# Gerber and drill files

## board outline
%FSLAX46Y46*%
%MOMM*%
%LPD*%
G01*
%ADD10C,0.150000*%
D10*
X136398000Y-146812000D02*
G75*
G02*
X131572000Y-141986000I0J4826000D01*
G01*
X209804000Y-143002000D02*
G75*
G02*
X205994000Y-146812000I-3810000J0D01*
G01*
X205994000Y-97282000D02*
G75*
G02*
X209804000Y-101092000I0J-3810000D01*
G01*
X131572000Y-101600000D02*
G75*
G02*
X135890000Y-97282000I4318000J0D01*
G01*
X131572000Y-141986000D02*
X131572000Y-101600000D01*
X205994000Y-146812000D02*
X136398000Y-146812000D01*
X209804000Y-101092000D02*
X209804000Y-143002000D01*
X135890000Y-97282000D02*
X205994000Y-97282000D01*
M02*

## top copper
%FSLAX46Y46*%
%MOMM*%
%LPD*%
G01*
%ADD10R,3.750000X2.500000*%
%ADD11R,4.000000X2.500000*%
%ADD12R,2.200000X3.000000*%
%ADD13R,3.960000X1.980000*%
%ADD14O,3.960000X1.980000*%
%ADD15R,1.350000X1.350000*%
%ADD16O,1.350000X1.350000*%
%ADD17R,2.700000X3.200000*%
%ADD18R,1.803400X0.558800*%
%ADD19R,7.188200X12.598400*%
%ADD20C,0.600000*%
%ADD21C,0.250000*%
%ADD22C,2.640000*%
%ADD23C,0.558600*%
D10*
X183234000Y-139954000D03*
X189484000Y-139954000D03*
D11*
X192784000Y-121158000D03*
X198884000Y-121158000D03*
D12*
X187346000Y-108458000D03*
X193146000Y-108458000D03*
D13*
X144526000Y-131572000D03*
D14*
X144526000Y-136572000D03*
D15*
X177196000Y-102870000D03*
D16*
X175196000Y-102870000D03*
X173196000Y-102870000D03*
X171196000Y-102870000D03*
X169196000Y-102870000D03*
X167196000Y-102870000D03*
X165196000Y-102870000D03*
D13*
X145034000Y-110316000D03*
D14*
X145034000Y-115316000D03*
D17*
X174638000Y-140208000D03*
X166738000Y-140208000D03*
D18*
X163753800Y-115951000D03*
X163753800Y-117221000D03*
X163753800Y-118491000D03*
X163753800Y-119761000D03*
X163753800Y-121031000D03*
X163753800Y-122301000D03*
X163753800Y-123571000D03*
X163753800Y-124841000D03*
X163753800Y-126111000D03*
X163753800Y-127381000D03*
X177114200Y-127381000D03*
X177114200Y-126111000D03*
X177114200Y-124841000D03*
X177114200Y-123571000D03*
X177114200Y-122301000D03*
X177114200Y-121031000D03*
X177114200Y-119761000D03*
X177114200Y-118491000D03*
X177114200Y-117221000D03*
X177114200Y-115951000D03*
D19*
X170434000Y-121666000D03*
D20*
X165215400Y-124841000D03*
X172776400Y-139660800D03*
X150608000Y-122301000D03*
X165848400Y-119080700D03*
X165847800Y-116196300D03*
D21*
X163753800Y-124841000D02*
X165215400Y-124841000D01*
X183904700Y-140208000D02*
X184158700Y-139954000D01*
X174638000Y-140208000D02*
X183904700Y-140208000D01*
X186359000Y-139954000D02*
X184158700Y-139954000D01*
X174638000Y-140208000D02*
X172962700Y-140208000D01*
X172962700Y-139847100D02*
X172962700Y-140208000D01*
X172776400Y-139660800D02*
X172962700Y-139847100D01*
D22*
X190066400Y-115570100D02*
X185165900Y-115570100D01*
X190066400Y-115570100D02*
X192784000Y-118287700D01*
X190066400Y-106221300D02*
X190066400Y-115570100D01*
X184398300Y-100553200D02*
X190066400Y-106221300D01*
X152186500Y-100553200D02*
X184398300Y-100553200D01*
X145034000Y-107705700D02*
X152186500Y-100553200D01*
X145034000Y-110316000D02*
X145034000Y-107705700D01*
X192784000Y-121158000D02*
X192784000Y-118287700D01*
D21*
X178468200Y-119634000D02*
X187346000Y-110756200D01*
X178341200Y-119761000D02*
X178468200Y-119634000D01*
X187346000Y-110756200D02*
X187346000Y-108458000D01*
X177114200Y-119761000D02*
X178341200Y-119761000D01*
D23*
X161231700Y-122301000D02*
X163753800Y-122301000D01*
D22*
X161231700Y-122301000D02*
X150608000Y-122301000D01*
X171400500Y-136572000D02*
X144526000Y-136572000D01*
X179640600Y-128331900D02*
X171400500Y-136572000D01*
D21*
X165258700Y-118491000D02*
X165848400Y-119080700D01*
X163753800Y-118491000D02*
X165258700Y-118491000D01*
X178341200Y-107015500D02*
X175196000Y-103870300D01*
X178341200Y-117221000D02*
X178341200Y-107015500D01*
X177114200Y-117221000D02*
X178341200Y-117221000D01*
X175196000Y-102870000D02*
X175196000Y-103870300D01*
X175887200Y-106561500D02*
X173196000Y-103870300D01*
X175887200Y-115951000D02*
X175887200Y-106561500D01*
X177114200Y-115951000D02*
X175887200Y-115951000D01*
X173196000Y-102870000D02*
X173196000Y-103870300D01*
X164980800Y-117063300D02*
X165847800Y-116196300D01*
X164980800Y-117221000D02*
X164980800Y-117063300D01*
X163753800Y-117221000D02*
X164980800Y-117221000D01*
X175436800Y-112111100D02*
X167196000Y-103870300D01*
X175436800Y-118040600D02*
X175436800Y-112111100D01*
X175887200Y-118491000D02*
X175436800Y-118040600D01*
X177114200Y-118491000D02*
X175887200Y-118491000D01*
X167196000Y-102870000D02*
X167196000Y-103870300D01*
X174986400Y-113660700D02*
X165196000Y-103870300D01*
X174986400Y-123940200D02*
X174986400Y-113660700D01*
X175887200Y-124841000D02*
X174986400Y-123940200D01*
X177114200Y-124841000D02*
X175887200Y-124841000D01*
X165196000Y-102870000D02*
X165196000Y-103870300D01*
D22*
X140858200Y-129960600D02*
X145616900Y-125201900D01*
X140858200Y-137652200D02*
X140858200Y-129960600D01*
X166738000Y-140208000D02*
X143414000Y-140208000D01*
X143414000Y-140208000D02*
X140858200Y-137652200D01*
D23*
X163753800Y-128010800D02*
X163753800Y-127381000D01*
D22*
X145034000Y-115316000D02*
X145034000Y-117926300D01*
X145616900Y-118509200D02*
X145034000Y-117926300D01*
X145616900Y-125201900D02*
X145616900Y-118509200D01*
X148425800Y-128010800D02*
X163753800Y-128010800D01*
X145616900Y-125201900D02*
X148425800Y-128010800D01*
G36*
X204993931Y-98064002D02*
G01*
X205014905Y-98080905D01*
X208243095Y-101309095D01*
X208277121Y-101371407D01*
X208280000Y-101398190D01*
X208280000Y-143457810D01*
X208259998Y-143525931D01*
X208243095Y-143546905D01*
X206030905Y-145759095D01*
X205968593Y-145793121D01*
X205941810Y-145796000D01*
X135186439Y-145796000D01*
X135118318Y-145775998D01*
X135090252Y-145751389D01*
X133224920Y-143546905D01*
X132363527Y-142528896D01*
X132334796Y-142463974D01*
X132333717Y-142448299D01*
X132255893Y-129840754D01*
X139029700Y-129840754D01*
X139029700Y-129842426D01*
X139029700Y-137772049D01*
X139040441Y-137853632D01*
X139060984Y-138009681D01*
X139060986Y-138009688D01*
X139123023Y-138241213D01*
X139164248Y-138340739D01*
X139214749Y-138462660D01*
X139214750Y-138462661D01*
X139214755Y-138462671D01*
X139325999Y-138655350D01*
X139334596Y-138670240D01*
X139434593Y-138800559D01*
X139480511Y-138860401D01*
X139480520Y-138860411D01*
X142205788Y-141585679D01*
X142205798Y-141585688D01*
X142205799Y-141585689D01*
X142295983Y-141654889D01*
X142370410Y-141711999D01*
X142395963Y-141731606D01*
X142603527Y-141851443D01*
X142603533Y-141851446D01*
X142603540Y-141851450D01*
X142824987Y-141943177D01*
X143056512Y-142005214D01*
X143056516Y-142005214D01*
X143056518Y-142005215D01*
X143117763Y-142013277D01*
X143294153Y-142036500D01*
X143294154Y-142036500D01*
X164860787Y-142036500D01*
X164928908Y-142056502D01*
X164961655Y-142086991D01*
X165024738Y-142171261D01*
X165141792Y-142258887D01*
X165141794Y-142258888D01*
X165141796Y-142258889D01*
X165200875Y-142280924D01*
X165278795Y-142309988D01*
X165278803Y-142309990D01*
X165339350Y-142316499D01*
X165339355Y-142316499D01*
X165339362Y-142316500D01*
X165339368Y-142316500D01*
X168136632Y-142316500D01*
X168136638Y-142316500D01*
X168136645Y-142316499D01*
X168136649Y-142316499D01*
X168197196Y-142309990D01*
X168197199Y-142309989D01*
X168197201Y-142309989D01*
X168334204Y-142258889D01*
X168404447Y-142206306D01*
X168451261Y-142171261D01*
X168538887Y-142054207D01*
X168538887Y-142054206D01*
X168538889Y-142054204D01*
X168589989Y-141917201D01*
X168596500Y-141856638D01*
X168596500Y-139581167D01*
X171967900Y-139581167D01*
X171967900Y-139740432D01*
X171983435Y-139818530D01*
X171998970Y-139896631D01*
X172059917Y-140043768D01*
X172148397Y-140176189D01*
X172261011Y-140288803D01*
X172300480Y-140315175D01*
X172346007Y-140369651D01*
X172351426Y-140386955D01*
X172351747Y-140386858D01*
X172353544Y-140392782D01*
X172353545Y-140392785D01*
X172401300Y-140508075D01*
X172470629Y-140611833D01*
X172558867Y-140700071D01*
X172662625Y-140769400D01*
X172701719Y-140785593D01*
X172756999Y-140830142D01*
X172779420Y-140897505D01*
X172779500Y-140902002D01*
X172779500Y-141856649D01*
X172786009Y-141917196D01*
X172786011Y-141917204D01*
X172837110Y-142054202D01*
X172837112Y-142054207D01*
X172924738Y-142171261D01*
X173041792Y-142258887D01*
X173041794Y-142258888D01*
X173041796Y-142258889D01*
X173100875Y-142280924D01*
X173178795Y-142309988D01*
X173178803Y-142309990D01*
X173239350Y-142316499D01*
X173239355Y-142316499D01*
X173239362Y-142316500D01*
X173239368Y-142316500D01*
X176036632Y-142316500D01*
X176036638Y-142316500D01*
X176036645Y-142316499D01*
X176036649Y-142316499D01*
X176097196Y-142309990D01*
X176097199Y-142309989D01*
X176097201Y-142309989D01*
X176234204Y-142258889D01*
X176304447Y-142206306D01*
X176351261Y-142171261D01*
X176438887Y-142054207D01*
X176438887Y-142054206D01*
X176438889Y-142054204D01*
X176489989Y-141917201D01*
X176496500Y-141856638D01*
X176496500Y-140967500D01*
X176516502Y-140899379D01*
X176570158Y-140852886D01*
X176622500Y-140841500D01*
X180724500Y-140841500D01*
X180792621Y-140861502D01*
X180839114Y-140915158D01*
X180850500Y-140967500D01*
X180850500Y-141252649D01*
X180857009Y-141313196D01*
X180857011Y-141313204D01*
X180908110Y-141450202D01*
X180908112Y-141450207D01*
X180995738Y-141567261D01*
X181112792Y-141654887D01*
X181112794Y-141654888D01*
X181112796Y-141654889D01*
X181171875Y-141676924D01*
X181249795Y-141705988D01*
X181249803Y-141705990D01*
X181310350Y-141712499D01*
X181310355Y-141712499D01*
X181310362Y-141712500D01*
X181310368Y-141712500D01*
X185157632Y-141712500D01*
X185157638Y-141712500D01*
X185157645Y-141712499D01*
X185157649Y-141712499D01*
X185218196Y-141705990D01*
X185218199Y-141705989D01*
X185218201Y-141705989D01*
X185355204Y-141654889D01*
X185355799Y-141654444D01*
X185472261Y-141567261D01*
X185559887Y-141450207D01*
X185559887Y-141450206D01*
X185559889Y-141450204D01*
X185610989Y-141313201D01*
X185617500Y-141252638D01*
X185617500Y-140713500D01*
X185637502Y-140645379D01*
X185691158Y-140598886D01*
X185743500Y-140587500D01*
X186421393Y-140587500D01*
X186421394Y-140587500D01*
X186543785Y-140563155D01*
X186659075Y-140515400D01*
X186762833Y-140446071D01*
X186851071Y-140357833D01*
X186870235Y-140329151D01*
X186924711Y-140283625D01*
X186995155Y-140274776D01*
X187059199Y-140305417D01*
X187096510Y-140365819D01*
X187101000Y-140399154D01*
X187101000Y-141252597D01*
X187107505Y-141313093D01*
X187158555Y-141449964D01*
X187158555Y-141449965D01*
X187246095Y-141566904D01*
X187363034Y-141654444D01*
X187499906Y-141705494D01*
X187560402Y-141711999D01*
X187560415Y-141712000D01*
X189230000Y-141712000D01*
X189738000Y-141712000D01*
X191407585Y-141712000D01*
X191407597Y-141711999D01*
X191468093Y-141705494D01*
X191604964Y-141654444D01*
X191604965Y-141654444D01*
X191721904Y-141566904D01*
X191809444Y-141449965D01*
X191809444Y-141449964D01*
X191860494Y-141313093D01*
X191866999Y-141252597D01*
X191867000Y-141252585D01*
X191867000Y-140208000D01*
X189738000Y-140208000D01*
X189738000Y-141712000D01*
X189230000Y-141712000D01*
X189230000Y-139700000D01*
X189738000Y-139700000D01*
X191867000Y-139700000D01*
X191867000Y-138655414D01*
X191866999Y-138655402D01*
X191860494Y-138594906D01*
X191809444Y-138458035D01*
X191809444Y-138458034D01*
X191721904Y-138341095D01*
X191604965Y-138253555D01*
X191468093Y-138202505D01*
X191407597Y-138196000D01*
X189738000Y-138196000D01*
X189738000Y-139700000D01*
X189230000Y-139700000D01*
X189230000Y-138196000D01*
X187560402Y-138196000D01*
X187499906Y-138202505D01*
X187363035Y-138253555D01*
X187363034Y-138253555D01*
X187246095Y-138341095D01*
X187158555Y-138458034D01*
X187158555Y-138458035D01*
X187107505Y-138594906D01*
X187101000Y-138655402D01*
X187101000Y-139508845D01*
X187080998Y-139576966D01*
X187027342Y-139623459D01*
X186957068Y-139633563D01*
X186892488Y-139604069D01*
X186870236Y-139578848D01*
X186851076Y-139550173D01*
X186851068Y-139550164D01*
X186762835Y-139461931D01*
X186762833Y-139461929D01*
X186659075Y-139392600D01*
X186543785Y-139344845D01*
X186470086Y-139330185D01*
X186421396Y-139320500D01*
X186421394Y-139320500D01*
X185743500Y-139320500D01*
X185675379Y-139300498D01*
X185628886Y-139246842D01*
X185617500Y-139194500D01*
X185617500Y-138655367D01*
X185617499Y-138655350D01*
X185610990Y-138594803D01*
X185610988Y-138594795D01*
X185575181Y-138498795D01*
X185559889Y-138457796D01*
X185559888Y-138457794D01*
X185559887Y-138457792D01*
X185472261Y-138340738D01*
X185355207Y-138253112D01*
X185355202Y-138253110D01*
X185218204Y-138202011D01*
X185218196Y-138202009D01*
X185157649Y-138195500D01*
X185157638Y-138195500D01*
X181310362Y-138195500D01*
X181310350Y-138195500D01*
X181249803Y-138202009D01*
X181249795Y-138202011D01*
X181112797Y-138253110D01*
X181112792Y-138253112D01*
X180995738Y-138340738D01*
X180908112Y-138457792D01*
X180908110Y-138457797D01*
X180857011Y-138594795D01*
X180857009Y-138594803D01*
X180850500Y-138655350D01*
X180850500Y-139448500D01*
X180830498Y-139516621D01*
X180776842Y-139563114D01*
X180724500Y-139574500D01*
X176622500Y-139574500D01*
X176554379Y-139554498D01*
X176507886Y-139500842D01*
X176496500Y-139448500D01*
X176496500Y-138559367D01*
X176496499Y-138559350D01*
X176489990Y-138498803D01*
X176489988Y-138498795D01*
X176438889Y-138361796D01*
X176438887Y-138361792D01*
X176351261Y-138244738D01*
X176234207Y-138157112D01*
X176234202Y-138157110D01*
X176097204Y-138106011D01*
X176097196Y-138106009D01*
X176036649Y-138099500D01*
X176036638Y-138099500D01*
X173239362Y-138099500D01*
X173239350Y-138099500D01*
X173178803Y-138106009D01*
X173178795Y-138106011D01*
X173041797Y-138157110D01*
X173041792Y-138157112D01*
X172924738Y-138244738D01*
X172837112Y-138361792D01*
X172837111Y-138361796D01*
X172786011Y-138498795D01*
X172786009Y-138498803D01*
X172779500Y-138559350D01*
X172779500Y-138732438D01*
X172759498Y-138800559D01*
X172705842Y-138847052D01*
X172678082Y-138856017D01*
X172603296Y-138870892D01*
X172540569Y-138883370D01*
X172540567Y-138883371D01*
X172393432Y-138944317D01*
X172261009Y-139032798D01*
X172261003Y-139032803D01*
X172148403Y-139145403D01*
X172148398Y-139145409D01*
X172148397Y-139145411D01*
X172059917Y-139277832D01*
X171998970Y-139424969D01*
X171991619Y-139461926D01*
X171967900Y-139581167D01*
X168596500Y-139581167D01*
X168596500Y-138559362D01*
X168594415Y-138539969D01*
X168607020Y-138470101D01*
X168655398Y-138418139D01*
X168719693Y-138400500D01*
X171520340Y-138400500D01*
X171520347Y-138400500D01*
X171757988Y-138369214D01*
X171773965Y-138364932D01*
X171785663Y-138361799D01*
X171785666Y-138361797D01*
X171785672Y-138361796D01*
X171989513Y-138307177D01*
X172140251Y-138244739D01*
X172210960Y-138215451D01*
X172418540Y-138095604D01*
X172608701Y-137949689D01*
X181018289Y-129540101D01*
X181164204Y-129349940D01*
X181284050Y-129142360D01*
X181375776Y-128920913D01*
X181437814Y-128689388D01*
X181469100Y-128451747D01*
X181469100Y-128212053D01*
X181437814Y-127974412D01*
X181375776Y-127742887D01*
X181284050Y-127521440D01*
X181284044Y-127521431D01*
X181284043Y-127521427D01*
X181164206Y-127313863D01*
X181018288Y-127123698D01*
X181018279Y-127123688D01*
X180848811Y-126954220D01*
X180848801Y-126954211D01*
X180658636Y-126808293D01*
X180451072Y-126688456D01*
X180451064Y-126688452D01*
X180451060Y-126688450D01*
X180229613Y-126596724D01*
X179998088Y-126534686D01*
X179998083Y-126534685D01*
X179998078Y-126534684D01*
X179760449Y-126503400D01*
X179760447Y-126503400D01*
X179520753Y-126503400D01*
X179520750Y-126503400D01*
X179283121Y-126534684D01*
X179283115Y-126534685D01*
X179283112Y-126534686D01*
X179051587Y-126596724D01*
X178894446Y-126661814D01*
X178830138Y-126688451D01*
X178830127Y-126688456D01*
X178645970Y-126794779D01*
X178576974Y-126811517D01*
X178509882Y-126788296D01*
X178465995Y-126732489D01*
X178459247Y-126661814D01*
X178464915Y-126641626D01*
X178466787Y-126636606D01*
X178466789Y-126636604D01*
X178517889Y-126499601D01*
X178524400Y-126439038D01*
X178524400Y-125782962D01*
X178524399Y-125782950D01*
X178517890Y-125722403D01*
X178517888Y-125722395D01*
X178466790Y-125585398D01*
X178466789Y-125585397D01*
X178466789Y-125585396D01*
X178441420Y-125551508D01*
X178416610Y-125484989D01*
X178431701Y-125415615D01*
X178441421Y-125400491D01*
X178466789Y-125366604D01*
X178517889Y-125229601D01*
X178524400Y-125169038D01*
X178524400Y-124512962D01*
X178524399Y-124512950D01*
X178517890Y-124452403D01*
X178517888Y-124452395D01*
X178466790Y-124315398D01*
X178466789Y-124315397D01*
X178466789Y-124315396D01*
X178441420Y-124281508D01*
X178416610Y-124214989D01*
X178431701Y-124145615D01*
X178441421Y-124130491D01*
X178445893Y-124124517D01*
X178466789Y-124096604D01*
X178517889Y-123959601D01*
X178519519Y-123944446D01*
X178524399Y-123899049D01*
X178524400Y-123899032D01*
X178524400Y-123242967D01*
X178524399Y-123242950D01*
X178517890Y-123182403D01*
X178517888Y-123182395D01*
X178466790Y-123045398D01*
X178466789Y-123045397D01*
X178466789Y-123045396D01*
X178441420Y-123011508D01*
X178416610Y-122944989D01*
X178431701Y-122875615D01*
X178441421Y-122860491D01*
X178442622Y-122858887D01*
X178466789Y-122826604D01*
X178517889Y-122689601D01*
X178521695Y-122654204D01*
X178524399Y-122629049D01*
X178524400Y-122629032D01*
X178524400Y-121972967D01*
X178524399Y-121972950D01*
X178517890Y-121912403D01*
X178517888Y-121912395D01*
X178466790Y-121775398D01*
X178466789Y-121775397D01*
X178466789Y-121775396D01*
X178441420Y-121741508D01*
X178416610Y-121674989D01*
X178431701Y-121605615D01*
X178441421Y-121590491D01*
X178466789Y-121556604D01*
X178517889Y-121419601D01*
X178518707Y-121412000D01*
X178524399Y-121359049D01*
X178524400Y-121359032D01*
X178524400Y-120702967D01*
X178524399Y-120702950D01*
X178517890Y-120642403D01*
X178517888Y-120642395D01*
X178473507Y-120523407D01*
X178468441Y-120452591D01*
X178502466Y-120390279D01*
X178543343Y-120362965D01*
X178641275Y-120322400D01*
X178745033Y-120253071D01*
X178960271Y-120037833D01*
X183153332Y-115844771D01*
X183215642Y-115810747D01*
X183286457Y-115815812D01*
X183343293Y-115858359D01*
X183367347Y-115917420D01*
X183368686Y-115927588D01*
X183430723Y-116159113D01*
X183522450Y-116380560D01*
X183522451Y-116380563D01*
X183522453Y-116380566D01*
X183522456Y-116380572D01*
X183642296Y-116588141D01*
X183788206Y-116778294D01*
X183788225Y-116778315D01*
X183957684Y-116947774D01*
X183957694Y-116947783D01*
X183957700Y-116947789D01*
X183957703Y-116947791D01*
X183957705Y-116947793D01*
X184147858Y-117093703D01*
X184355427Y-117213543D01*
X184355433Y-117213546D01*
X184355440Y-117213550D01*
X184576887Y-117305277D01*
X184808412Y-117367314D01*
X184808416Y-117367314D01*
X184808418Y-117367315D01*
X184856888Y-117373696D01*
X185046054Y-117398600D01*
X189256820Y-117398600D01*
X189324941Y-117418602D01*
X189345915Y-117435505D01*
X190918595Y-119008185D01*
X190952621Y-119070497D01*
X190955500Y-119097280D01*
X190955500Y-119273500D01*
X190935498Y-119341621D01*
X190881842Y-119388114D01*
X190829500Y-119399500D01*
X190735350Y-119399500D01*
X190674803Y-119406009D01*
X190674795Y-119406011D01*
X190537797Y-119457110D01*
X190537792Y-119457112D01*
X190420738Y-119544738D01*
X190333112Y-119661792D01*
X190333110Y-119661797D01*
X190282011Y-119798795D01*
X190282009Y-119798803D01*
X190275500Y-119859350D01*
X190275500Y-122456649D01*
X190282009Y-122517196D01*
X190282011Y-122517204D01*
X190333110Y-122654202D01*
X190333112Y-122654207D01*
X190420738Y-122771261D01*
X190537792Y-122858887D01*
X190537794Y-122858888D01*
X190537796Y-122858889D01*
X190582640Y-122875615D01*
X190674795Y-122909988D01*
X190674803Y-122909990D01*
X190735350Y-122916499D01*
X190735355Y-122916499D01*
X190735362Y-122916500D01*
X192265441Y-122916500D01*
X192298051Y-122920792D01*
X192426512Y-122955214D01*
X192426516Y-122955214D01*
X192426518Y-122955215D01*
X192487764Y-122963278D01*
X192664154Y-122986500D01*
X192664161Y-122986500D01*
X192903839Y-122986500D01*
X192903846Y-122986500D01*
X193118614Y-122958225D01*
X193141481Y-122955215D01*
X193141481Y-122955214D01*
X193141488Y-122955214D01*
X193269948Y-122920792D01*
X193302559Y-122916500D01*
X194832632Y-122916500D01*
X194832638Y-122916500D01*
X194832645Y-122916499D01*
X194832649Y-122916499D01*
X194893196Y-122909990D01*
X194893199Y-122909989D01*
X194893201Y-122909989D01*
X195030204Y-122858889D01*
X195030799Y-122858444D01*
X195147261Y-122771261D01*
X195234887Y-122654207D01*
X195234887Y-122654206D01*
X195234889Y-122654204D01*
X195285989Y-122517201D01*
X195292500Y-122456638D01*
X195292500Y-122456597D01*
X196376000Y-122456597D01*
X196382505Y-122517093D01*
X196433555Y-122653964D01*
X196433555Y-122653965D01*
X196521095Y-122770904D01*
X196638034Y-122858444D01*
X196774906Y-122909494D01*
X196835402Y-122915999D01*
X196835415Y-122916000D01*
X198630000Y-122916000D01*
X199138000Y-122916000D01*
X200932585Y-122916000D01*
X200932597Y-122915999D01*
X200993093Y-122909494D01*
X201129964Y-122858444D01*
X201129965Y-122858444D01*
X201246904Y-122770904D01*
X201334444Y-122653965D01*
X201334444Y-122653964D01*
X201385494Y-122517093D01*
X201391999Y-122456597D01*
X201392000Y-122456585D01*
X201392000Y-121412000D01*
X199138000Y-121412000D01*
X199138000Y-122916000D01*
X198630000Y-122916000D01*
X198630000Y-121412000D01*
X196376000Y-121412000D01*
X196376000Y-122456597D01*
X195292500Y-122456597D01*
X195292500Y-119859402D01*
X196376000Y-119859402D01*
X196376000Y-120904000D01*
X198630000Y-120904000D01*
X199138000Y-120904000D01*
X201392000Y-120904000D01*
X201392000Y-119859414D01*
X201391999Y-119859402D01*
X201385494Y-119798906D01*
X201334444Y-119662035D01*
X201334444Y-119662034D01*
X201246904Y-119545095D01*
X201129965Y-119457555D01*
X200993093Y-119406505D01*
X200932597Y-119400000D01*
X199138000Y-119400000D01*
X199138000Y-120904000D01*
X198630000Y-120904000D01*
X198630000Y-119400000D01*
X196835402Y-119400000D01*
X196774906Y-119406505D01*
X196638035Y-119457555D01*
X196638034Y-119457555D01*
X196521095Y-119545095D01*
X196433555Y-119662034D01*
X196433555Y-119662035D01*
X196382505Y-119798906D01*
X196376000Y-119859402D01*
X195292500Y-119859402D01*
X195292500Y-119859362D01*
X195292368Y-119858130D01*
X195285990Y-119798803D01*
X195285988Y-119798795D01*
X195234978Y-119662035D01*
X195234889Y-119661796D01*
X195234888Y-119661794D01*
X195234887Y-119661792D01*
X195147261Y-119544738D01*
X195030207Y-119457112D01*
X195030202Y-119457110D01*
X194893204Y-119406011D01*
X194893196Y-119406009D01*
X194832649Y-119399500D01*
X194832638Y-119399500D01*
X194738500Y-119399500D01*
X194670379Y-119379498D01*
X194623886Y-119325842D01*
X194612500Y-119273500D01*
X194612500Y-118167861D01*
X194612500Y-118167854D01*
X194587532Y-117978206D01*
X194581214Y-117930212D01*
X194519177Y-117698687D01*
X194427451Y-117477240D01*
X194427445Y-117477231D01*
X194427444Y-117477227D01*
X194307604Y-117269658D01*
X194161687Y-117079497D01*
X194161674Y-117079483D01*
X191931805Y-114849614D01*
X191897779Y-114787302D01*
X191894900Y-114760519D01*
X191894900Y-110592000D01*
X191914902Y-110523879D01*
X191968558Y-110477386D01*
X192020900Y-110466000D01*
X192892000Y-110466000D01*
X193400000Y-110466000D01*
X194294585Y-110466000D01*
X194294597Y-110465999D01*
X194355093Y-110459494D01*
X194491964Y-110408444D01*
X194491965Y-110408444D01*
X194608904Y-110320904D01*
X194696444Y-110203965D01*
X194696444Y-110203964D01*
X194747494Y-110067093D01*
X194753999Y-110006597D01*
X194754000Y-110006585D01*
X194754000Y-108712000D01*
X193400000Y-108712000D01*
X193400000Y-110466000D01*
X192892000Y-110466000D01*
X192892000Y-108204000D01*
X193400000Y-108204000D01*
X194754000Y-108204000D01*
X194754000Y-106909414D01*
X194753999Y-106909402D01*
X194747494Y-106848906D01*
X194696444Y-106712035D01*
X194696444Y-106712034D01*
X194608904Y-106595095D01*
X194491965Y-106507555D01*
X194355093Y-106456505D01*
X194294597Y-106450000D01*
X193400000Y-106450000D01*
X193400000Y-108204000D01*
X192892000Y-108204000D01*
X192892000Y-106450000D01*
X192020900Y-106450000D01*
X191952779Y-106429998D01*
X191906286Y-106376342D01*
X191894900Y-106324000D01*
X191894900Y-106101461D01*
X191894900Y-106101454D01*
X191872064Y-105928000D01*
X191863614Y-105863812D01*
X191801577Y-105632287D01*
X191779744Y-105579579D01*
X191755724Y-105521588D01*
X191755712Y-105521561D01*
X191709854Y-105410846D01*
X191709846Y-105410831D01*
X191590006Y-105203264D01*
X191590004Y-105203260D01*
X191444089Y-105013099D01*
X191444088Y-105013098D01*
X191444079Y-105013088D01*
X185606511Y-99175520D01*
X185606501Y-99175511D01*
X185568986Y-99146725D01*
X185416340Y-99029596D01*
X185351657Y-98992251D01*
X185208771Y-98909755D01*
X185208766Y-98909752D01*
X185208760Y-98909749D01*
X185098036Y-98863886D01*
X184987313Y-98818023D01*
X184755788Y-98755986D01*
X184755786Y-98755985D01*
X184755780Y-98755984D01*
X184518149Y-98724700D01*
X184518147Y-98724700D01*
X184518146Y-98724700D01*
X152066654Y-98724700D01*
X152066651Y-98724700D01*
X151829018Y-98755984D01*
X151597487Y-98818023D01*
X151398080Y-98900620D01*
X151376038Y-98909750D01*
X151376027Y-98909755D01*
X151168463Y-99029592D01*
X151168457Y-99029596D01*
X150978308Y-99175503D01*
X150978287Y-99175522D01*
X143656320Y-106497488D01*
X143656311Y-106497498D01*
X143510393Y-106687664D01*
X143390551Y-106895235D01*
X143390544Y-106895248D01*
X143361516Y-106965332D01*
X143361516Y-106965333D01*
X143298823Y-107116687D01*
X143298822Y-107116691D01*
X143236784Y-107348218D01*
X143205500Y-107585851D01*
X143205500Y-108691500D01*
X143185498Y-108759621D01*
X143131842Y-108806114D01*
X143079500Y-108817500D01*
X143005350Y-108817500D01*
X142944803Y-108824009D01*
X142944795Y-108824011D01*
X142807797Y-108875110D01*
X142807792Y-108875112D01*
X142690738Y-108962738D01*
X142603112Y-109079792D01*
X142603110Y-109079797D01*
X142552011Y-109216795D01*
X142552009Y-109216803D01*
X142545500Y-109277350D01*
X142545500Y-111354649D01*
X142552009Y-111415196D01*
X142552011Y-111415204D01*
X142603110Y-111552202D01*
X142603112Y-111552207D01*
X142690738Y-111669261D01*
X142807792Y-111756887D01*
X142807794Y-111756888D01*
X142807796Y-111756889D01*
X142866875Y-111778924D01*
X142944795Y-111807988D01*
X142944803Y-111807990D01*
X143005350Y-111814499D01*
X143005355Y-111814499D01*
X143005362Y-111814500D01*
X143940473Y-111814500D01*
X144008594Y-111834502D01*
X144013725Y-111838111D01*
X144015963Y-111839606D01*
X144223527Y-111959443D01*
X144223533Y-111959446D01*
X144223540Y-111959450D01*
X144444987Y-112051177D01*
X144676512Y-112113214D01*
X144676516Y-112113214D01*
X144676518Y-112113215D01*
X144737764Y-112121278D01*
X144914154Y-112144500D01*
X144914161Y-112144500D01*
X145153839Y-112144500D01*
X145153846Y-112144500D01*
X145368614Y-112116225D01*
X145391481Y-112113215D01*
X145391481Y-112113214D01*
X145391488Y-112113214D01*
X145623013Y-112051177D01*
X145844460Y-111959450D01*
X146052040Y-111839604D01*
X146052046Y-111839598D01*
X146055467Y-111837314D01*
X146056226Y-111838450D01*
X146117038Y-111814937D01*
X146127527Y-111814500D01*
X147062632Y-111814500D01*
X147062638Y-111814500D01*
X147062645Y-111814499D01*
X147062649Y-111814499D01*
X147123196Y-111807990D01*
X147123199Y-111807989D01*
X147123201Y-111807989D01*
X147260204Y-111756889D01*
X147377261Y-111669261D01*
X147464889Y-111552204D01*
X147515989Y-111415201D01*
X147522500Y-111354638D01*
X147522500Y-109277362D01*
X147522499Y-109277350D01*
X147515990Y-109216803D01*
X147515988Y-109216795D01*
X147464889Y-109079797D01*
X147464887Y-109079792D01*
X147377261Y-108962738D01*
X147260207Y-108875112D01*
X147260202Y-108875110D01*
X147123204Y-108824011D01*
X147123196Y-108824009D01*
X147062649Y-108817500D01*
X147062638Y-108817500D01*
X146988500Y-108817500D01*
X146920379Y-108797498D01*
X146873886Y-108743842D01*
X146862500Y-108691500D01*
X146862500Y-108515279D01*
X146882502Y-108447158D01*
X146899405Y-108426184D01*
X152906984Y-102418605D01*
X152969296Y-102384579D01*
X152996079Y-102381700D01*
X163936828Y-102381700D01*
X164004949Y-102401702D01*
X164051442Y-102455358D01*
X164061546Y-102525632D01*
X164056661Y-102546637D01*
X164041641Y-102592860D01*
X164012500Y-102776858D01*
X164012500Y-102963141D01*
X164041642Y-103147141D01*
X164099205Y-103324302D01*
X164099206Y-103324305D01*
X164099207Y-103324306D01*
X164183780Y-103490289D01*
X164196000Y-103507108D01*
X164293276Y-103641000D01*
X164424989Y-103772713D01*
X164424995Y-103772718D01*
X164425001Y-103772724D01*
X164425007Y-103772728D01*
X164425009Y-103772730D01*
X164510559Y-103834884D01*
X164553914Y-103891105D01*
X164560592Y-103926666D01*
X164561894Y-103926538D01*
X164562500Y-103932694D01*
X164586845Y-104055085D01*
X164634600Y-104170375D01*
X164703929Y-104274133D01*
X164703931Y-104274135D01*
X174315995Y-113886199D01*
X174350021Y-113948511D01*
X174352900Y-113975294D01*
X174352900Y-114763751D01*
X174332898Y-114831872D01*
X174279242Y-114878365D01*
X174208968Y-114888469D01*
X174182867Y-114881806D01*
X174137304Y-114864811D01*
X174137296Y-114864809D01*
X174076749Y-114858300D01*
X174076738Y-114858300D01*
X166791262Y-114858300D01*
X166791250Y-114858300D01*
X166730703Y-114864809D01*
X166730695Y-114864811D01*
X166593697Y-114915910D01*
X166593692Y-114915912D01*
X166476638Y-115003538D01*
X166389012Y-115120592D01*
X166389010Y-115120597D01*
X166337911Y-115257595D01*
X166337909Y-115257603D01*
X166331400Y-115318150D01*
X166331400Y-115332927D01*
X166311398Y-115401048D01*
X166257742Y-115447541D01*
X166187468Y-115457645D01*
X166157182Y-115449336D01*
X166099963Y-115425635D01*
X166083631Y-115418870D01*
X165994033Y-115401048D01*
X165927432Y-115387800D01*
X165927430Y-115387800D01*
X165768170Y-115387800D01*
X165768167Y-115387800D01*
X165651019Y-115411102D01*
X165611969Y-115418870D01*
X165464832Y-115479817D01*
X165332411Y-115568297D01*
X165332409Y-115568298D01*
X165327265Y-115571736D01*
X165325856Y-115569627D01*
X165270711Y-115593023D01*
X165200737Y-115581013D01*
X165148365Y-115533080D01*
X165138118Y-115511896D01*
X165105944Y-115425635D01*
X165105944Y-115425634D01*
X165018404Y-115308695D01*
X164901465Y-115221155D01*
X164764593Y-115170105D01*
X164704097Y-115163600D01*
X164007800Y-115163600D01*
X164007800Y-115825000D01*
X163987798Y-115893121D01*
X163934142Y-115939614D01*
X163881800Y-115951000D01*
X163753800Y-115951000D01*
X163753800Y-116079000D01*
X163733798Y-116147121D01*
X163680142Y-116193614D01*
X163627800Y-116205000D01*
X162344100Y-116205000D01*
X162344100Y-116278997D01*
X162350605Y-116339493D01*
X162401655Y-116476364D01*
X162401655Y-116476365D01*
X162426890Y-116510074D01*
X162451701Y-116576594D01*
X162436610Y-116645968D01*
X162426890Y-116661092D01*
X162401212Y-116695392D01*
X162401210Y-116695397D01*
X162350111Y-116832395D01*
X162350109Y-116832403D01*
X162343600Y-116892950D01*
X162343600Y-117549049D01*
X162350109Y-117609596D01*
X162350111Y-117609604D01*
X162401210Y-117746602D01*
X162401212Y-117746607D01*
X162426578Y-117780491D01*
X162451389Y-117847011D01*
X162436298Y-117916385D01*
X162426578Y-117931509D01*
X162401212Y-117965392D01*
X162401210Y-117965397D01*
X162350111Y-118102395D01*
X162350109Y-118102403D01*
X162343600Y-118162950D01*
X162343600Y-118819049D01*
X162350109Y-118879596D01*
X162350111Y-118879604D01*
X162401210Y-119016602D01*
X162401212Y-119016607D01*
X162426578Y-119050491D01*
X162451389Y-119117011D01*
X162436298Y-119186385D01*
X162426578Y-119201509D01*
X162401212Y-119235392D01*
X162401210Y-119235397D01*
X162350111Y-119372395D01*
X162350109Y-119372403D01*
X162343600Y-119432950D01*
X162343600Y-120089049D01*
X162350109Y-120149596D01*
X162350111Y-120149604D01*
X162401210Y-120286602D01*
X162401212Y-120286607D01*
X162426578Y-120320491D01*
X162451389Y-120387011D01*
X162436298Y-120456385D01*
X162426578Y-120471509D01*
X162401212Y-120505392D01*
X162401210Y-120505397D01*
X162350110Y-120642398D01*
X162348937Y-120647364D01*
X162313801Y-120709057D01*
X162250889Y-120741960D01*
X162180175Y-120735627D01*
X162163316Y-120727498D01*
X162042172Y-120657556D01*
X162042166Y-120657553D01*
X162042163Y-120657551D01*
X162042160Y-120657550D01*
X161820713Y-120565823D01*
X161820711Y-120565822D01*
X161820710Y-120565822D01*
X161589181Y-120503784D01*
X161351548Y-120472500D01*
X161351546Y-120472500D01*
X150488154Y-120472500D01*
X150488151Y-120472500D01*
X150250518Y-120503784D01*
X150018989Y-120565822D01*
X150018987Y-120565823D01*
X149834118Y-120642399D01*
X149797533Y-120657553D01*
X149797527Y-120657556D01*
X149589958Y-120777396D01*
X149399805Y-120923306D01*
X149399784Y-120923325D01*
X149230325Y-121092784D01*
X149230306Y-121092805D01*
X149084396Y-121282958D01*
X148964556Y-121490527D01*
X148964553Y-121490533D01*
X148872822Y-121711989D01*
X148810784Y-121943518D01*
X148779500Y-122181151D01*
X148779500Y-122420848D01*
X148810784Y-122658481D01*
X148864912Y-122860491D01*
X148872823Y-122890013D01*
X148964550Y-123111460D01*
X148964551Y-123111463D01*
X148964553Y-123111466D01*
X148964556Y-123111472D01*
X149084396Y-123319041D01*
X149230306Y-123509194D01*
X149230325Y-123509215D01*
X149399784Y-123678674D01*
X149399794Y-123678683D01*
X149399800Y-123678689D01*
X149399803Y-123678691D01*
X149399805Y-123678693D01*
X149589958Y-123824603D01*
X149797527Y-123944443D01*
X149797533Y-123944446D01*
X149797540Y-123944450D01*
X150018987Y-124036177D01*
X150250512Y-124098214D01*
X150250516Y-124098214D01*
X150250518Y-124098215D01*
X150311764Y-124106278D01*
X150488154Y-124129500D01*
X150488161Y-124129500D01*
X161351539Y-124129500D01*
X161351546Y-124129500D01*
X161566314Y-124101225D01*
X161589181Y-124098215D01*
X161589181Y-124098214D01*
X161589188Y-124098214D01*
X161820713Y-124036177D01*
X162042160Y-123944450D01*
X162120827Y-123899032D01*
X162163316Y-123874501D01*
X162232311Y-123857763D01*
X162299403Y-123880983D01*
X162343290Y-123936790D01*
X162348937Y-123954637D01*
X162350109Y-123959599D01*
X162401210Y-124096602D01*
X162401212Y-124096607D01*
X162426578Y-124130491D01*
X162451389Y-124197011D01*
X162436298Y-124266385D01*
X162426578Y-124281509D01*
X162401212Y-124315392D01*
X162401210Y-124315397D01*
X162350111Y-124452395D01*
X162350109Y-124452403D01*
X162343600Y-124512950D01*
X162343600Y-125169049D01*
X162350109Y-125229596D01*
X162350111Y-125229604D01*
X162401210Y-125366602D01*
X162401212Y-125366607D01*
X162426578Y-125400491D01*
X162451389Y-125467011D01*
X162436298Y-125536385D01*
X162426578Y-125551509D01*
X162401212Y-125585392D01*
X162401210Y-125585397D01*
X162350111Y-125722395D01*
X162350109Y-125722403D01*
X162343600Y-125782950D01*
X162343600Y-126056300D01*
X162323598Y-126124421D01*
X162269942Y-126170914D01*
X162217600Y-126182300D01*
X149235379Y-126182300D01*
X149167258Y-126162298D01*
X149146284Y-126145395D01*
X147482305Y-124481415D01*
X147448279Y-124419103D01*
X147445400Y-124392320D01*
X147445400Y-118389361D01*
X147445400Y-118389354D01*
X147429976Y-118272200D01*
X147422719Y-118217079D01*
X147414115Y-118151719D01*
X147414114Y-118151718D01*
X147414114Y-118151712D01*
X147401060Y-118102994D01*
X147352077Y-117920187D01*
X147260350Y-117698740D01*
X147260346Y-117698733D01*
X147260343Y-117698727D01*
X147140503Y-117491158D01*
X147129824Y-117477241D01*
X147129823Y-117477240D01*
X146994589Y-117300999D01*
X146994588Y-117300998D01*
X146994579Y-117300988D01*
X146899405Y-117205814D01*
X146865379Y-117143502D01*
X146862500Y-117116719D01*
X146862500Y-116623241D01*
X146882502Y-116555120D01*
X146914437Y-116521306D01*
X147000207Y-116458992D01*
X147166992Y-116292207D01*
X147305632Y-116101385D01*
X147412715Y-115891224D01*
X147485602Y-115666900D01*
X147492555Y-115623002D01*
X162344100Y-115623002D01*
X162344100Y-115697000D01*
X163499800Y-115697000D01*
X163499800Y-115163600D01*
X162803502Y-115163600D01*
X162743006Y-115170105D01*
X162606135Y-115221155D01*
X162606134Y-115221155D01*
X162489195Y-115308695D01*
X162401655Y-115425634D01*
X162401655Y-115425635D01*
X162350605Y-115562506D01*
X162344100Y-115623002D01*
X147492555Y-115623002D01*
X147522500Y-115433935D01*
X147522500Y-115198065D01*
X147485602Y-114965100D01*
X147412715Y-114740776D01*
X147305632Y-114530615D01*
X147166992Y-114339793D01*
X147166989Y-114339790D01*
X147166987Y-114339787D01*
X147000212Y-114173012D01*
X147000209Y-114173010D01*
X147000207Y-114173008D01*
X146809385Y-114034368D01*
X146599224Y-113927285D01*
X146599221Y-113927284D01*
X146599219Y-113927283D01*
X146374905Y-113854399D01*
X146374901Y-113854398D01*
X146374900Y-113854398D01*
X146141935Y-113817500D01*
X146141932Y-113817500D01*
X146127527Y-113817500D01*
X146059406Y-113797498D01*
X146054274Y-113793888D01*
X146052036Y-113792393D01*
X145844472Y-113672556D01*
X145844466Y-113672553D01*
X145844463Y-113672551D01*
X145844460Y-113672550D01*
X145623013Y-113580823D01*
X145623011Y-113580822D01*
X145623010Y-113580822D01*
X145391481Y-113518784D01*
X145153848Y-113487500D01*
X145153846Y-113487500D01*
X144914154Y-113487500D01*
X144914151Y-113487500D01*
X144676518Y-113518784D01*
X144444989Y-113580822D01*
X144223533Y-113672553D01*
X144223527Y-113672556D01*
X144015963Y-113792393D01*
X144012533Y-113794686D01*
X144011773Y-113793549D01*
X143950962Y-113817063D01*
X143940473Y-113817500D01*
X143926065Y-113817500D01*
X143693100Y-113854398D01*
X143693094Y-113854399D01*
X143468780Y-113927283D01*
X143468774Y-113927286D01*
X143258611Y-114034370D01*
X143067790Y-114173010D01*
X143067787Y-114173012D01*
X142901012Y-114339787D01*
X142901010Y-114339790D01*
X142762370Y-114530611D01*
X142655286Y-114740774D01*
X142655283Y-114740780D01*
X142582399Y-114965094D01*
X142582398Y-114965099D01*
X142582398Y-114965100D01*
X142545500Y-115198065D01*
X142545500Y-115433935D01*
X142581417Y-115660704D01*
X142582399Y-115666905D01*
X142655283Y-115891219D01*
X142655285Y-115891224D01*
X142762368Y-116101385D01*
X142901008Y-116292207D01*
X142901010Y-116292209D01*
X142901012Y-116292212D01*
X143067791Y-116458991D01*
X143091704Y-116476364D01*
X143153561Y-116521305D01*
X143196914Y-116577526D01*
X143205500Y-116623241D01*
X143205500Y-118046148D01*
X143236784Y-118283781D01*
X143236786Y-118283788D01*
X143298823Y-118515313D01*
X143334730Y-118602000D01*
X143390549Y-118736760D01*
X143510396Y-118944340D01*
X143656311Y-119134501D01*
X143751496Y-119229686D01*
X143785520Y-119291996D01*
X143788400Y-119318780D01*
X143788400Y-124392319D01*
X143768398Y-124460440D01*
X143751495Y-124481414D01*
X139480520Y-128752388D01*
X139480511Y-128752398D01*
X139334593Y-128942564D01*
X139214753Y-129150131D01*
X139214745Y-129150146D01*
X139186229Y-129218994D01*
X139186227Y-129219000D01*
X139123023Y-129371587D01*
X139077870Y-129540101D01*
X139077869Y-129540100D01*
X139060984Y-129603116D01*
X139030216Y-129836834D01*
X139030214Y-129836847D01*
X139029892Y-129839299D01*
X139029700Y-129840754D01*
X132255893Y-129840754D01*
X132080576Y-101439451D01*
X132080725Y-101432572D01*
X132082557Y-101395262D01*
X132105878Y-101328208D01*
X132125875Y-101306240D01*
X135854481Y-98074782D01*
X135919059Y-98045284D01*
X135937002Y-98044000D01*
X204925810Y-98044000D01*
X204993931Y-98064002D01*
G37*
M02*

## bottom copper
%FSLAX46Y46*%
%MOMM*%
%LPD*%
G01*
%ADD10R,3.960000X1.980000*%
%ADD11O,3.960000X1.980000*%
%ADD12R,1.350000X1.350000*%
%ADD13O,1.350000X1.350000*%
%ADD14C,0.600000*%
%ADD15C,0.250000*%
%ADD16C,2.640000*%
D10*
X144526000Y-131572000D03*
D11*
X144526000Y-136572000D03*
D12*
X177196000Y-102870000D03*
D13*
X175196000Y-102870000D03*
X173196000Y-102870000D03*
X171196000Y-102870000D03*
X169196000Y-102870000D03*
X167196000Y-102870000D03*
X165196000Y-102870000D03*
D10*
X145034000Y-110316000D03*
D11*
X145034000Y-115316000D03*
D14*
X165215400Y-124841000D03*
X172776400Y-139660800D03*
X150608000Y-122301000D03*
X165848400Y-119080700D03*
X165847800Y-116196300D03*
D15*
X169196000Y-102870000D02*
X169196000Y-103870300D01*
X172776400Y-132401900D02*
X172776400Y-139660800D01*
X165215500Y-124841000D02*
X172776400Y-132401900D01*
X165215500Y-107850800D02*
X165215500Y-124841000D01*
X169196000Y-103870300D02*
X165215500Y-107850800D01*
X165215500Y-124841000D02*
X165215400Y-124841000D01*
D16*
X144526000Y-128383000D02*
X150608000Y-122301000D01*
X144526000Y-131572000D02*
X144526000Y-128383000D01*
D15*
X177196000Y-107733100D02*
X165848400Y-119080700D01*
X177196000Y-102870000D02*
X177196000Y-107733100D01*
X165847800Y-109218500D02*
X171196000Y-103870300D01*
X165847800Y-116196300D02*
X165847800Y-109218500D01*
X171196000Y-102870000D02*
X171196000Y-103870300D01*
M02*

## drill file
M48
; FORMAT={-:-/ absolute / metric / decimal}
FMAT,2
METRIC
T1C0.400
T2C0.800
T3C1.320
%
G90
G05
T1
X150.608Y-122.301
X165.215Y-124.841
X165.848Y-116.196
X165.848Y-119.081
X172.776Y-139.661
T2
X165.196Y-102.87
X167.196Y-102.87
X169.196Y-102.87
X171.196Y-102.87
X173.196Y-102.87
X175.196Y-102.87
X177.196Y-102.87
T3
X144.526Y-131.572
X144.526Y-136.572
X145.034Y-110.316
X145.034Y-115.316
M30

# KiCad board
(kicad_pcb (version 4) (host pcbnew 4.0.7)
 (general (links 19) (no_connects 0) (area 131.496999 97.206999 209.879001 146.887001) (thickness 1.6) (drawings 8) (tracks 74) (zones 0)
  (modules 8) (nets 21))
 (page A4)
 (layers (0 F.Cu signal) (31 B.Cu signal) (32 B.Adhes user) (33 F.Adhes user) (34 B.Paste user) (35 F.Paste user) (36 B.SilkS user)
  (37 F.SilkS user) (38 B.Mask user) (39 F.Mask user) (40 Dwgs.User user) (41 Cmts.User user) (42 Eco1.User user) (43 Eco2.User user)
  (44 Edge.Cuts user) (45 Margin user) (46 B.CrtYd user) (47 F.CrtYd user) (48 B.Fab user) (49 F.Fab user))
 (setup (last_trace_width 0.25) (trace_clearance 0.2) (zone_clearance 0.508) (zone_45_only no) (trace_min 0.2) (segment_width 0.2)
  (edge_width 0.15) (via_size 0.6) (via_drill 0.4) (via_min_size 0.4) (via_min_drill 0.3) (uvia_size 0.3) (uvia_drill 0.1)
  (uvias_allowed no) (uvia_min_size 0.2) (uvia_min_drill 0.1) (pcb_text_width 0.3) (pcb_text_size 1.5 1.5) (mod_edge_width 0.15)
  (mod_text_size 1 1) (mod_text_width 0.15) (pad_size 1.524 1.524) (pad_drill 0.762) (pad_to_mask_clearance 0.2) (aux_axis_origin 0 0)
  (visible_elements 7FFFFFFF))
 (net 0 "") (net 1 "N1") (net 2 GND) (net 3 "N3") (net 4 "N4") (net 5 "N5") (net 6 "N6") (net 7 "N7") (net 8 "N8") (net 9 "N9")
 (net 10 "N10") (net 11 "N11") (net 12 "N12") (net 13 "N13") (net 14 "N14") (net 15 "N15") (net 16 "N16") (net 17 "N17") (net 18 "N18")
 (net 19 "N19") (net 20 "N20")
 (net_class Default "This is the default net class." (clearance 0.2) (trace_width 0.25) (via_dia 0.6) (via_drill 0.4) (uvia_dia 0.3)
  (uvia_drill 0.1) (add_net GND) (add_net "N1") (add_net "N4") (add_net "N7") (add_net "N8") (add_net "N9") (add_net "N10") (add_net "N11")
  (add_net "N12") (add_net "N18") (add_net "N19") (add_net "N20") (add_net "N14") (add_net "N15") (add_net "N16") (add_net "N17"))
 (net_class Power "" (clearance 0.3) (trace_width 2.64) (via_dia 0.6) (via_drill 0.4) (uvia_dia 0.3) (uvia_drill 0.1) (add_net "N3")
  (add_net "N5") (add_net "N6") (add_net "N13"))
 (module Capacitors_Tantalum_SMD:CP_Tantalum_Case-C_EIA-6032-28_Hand (layer F.Cu) (at 186.359 139.954)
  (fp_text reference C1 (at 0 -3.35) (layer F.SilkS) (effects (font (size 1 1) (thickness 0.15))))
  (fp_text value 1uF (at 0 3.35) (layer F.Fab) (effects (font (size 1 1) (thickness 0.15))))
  (pad 1 smd rect (at -3.125 0) (size 3.75 2.5) (layers F.Cu F.Paste F.Mask) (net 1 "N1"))
  (pad 2 smd rect (at 3.125 0) (size 3.75 2.5) (layers F.Cu F.Paste F.Mask) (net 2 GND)))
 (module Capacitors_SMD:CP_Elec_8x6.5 (layer F.Cu) (at 195.834 121.158)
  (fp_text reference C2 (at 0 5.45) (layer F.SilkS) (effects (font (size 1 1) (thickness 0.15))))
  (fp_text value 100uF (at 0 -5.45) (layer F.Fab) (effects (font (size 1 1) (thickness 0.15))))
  (pad 1 smd rect (at -3.05 0 180) (size 4 2.5) (layers F.Cu F.Paste F.Mask) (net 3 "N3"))
  (pad 2 smd rect (at 3.05 0 180) (size 4 2.5) (layers F.Cu F.Paste F.Mask) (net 2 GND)))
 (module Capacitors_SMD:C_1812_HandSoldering (layer F.Cu) (at 190.246 108.458)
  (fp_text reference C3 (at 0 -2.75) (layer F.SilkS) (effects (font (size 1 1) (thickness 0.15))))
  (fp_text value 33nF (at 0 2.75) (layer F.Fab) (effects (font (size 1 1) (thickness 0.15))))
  (pad 1 smd rect (at -2.9 0) (size 2.2 3) (layers F.Cu F.Paste F.Mask) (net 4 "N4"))
  (pad 2 smd rect (at 2.9 0) (size 2.2 3) (layers F.Cu F.Paste F.Mask) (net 2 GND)))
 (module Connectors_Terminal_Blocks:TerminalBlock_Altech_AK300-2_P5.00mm (layer F.Cu) (at 144.526 131.572 270)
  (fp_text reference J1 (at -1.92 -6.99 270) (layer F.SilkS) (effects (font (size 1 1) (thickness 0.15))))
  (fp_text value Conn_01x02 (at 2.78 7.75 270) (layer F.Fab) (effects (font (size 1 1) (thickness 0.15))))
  (pad 1 thru_hole rect (at 0 0 270) (size 1.98 3.96) (drill 1.32) (layers *.Cu *.Mask) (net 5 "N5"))
  (pad 2 thru_hole oval (at 5 0 270) (size 1.98 3.96) (drill 1.32) (layers *.Cu *.Mask) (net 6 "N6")))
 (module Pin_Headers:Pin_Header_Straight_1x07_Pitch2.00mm (layer F.Cu) (at 177.196 102.87 270)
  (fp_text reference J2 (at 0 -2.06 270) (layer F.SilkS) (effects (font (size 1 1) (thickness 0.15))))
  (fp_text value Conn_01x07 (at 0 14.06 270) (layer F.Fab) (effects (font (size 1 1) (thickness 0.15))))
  (pad 1 thru_hole rect (at 0 0 270) (size 1.35 1.35) (drill 0.8) (layers *.Cu *.Mask) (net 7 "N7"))
  (pad 2 thru_hole oval (at 0 2 270) (size 1.35 1.35) (drill 0.8) (layers *.Cu *.Mask) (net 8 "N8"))
  (pad 3 thru_hole oval (at 0 4 270) (size 1.35 1.35) (drill 0.8) (layers *.Cu *.Mask) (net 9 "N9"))
  (pad 4 thru_hole oval (at 0 6 270) (size 1.35 1.35) (drill 0.8) (layers *.Cu *.Mask) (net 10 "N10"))
  (pad 5 thru_hole oval (at 0 8 270) (size 1.35 1.35) (drill 0.8) (layers *.Cu *.Mask) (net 1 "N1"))
  (pad 6 thru_hole oval (at 0 10 270) (size 1.35 1.35) (drill 0.8) (layers *.Cu *.Mask) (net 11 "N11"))
  (pad 7 thru_hole oval (at 0 12 270) (size 1.35 1.35) (drill 0.8) (layers *.Cu *.Mask) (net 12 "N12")))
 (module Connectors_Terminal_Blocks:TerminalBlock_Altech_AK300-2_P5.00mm (layer F.Cu) (at 145.034 110.316 270)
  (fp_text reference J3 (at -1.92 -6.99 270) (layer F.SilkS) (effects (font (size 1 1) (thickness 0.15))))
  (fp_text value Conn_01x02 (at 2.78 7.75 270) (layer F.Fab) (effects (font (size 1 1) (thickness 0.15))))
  (pad 1 thru_hole rect (at 0 0 270) (size 1.98 3.96) (drill 1.32) (layers *.Cu *.Mask) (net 3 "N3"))
  (pad 2 thru_hole oval (at 5 0 270) (size 1.98 3.96) (drill 1.32) (layers *.Cu *.Mask) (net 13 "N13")))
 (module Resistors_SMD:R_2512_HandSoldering (layer F.Cu) (at 170.688 140.208 180)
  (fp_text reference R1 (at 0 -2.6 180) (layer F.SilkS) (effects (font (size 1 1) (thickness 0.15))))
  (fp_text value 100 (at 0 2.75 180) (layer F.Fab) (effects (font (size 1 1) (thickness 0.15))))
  (pad 1 smd rect (at -3.95 0 180) (size 2.7 3.2) (layers F.Cu F.Paste F.Mask) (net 1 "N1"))
  (pad 2 smd rect (at 3.95 0 180) (size 2.7 3.2) (layers F.Cu F.Paste F.Mask) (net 13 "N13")))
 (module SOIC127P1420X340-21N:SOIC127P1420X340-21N (layer F.Cu) (at 170.434 121.666)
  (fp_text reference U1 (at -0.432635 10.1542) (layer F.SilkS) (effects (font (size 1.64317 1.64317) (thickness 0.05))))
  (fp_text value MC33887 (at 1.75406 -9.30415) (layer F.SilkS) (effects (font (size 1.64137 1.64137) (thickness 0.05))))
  (pad 1 smd rect (at -6.6802 -5.715) (size 1.8034 0.5588) (layers F.Cu F.Paste F.Mask) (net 2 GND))
  (pad 2 smd rect (at -6.6802 -4.445) (size 1.8034 0.5588) (layers F.Cu F.Paste F.Mask) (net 10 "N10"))
  (pad 3 smd rect (at -6.6802 -3.175) (size 1.8034 0.5588) (layers F.Cu F.Paste F.Mask) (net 7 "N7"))
  (pad 4 smd rect (at -6.6802 -1.905) (size 1.8034 0.5588) (layers F.Cu F.Paste F.Mask) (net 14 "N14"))
  (pad 5 smd rect (at -6.6802 -0.635) (size 1.8034 0.5588) (layers F.Cu F.Paste F.Mask) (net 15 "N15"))
  (pad 6 smd rect (at -6.6802 0.635) (size 1.8034 0.5588) (layers F.Cu F.Paste F.Mask) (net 5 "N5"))
  (pad 7 smd rect (at -6.6802 1.905) (size 1.8034 0.5588) (layers F.Cu F.Paste F.Mask) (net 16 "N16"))
  (pad 8 smd rect (at -6.6802 3.175) (size 1.8034 0.5588) (layers F.Cu F.Paste F.Mask) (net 1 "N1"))
  (pad 9 smd rect (at -6.6802 4.445) (size 1.8034 0.5588) (layers F.Cu F.Paste F.Mask) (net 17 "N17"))
  (pad 10 smd rect (at -6.6802 5.715) (size 1.8034 0.5588) (layers F.Cu F.Paste F.Mask) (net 13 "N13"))
  (pad 11 smd rect (at 6.6802 5.715) (size 1.8034 0.5588) (layers F.Cu F.Paste F.Mask) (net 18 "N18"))
  (pad 12 smd rect (at 6.6802 4.445) (size 1.8034 0.5588) (layers F.Cu F.Paste F.Mask) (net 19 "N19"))
  (pad 13 smd rect (at 6.6802 3.175) (size 1.8034 0.5588) (layers F.Cu F.Paste F.Mask) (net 12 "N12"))
  (pad 14 smd rect (at 6.6802 1.905) (size 1.8034 0.5588) (layers F.Cu F.Paste F.Mask) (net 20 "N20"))
  (pad 15 smd rect (at 6.6802 0.635) (size 1.8034 0.5588) (layers F.Cu F.Paste F.Mask) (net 6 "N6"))
  (pad 16 smd rect (at 6.6802 -0.635) (size 1.8034 0.5588) (layers F.Cu F.Paste F.Mask) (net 3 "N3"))
  (pad 17 smd rect (at 6.6802 -1.905) (size 1.8034 0.5588) (layers F.Cu F.Paste F.Mask) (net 4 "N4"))
  (pad 18 smd rect (at 6.6802 -3.175) (size 1.8034 0.5588) (layers F.Cu F.Paste F.Mask) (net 11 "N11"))
  (pad 19 smd rect (at 6.6802 -4.445) (size 1.8034 0.5588) (layers F.Cu F.Paste F.Mask) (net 8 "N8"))
  (pad 20 smd rect (at 6.6802 -5.715) (size 1.8034 0.5588) (layers F.Cu F.Paste F.Mask) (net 9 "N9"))
  (pad 21 smd rect (at 0 0) (size 7.1882 12.5984) (layers F.Cu F.Paste F.Mask)))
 (gr_arc (start 136.398 141.986) (end 136.398 146.812) (angle 90) (layer Edge.Cuts) (width 0.15))
 (gr_arc (start 205.994 143.002) (end 209.804 143.002) (angle 90) (layer Edge.Cuts) (width 0.15))
 (gr_arc (start 205.994 101.092) (end 205.994 97.282) (angle 90) (layer Edge.Cuts) (width 0.15))
 (gr_arc (start 135.89 101.6) (end 131.572 101.6) (angle 90) (layer Edge.Cuts) (width 0.15))
 (gr_line (start 131.572 141.986) (end 131.572 101.6) (layer Edge.Cuts) (width 0.15))
 (gr_line (start 205.994 146.812) (end 136.398 146.812) (layer Edge.Cuts) (width 0.15))
 (gr_line (start 209.804 101.092) (end 209.804 143.002) (layer Edge.Cuts) (width 0.15))
 (gr_line (start 135.89 97.282) (end 205.994 97.282) (layer Edge.Cuts) (width 0.15))
 (via (at 165.2154 124.841) (size 0.6) (layers F.Cu B.Cu) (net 1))
 (via (at 172.7764 139.6608) (size 0.6) (layers F.Cu B.Cu) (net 1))
 (segment (start 169.196 102.87) (end 169.196 103.8703) (width 0.25) (layer B.Cu) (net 1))
 (segment (start 163.7538 124.841) (end 165.2154 124.841) (width 0.25) (layer F.Cu) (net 1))
 (segment (start 183.9047 140.208) (end 184.1587 139.954) (width 0.25) (layer F.Cu) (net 1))
 (segment (start 174.638 140.208) (end 183.9047 140.208) (width 0.25) (layer F.Cu) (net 1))
 (segment (start 186.359 139.954) (end 184.1587 139.954) (width 0.25) (layer F.Cu) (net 1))
 (segment (start 174.638 140.208) (end 172.9627 140.208) (width 0.25) (layer F.Cu) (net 1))
 (segment (start 172.9627 139.8471) (end 172.9627 140.208) (width 0.25) (layer F.Cu) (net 1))
 (segment (start 172.7764 139.6608) (end 172.9627 139.8471) (width 0.25) (layer F.Cu) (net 1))
 (segment (start 172.7764 132.4019) (end 172.7764 139.6608) (width 0.25) (layer B.Cu) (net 1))
 (segment (start 165.2155 124.841) (end 172.7764 132.4019) (width 0.25) (layer B.Cu) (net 1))
 (segment (start 165.2155 107.8508) (end 165.2155 124.841) (width 0.25) (layer B.Cu) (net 1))
 (segment (start 169.196 103.8703) (end 165.2155 107.8508) (width 0.25) (layer B.Cu) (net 1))
 (segment (start 165.2155 124.841) (end 165.2154 124.841) (width 0.25) (layer B.Cu) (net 1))
 (segment (start 190.0664 115.5701) (end 185.1659 115.5701) (width 2.64) (layer F.Cu) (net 3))
 (segment (start 190.0664 115.5701) (end 192.784 118.2877) (width 2.64) (layer F.Cu) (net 3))
 (segment (start 190.0664 106.2213) (end 190.0664 115.5701) (width 2.64) (layer F.Cu) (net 3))
 (segment (start 184.3983 100.5532) (end 190.0664 106.2213) (width 2.64) (layer F.Cu) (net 3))
 (segment (start 152.1865 100.5532) (end 184.3983 100.5532) (width 2.64) (layer F.Cu) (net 3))
 (segment (start 145.034 107.7057) (end 152.1865 100.5532) (width 2.64) (layer F.Cu) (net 3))
 (segment (start 145.034 110.316) (end 145.034 107.7057) (width 2.64) (layer F.Cu) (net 3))
 (segment (start 192.784 121.158) (end 192.784 118.2877) (width 2.64) (layer F.Cu) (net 3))
 (segment (start 178.4682 119.634) (end 187.346 110.7562) (width 0.25) (layer F.Cu) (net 4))
 (segment (start 178.3412 119.761) (end 178.4682 119.634) (width 0.25) (layer F.Cu) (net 4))
 (segment (start 187.346 110.7562) (end 187.346 108.458) (width 0.25) (layer F.Cu) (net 4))
 (segment (start 177.1142 119.761) (end 178.3412 119.761) (width 0.25) (layer F.Cu) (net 4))
 (via (at 150.608 122.301) (size 0.6) (layers F.Cu B.Cu) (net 5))
 (segment (start 161.2317 122.301) (end 163.7538 122.301) (width 0.5586) (layer F.Cu) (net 5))
 (segment (start 144.526 128.383) (end 150.608 122.301) (width 2.64) (layer B.Cu) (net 5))
 (segment (start 144.526 131.572) (end 144.526 128.383) (width 2.64) (layer B.Cu) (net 5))
 (segment (start 161.2317 122.301) (end 150.608 122.301) (width 2.64) (layer F.Cu) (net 5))
 (segment (start 171.4005 136.572) (end 144.526 136.572) (width 2.64) (layer F.Cu) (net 6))
 (segment (start 179.6406 128.3319) (end 171.4005 136.572) (width 2.64) (layer F.Cu) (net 6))
 (via (at 165.8484 119.0807) (size 0.6) (layers F.Cu B.Cu) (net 7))
 (segment (start 177.196 107.7331) (end 165.8484 119.0807) (width 0.25) (layer B.Cu) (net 7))
 (segment (start 177.196 102.87) (end 177.196 107.7331) (width 0.25) (layer B.Cu) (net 7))
 (segment (start 165.2587 118.491) (end 165.8484 119.0807) (width 0.25) (layer F.Cu) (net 7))
 (segment (start 163.7538 118.491) (end 165.2587 118.491) (width 0.25) (layer F.Cu) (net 7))
 (segment (start 178.3412 107.0155) (end 175.196 103.8703) (width 0.25) (layer F.Cu) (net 8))
 (segment (start 178.3412 117.221) (end 178.3412 107.0155) (width 0.25) (layer F.Cu) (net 8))
 (segment (start 177.1142 117.221) (end 178.3412 117.221) (width 0.25) (layer F.Cu) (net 8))
 (segment (start 175.196 102.87) (end 175.196 103.8703) (width 0.25) (layer F.Cu) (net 8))
 (segment (start 175.8872 106.5615) (end 173.196 103.8703) (width 0.25) (layer F.Cu) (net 9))
 (segment (start 175.8872 115.951) (end 175.8872 106.5615) (width 0.25) (layer F.Cu) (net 9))
 (segment (start 177.1142 115.951) (end 175.8872 115.951) (width 0.25) (layer F.Cu) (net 9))
 (segment (start 173.196 102.87) (end 173.196 103.8703) (width 0.25) (layer F.Cu) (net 9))
 (via (at 165.8478 116.1963) (size 0.6) (layers F.Cu B.Cu) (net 10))
 (segment (start 164.9808 117.0633) (end 165.8478 116.1963) (width 0.25) (layer F.Cu) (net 10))
 (segment (start 164.9808 117.221) (end 164.9808 117.0633) (width 0.25) (layer F.Cu) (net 10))
 (segment (start 165.8478 109.2185) (end 171.196 103.8703) (width 0.25) (layer B.Cu) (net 10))
 (segment (start 165.8478 116.1963) (end 165.8478 109.2185) (width 0.25) (layer B.Cu) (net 10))
 (segment (start 163.7538 117.221) (end 164.9808 117.221) (width 0.25) (layer F.Cu) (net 10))
 (segment (start 171.196 102.87) (end 171.196 103.8703) (width 0.25) (layer B.Cu) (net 10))
 (segment (start 175.4368 112.1111) (end 167.196 103.8703) (width 0.25) (layer F.Cu) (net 11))
 (segment (start 175.4368 118.0406) (end 175.4368 112.1111) (width 0.25) (layer F.Cu) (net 11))
 (segment (start 175.8872 118.491) (end 175.4368 118.0406) (width 0.25) (layer F.Cu) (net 11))
 (segment (start 177.1142 118.491) (end 175.8872 118.491) (width 0.25) (layer F.Cu) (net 11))
 (segment (start 167.196 102.87) (end 167.196 103.8703) (width 0.25) (layer F.Cu) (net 11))
 (segment (start 174.9864 113.6607) (end 165.196 103.8703) (width 0.25) (layer F.Cu) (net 12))
 (segment (start 174.9864 123.9402) (end 174.9864 113.6607) (width 0.25) (layer F.Cu) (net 12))
 (segment (start 175.8872 124.841) (end 174.9864 123.9402) (width 0.25) (layer F.Cu) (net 12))
 (segment (start 177.1142 124.841) (end 175.8872 124.841) (width 0.25) (layer F.Cu) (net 12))
 (segment (start 165.196 102.87) (end 165.196 103.8703) (width 0.25) (layer F.Cu) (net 12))
 (segment (start 140.8582 129.9606) (end 145.6169 125.2019) (width 2.64) (layer F.Cu) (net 13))
 (segment (start 140.8582 137.6522) (end 140.8582 129.9606) (width 2.64) (layer F.Cu) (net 13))
 (segment (start 166.738 140.208) (end 143.414 140.208) (width 2.64) (layer F.Cu) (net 13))
 (segment (start 143.414 140.208) (end 140.8582 137.6522) (width 2.64) (layer F.Cu) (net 13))
 (segment (start 163.7538 128.0108) (end 163.7538 127.381) (width 0.5586) (layer F.Cu) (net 13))
 (segment (start 145.034 115.316) (end 145.034 117.9263) (width 2.64) (layer F.Cu) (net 13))
 (segment (start 145.6169 118.5092) (end 145.034 117.9263) (width 2.64) (layer F.Cu) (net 13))
 (segment (start 145.6169 125.2019) (end 145.6169 118.5092) (width 2.64) (layer F.Cu) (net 13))
 (segment (start 148.4258 128.0108) (end 163.7538 128.0108) (width 2.64) (layer F.Cu) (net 13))
 (segment (start 145.6169 125.2019) (end 148.4258 128.0108) (width 2.64) (layer F.Cu) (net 13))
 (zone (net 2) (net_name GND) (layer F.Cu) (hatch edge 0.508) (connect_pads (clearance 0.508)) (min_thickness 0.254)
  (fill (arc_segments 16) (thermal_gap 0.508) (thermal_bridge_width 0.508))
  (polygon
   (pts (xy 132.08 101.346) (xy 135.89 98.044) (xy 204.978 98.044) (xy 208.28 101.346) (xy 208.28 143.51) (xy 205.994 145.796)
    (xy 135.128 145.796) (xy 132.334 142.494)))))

